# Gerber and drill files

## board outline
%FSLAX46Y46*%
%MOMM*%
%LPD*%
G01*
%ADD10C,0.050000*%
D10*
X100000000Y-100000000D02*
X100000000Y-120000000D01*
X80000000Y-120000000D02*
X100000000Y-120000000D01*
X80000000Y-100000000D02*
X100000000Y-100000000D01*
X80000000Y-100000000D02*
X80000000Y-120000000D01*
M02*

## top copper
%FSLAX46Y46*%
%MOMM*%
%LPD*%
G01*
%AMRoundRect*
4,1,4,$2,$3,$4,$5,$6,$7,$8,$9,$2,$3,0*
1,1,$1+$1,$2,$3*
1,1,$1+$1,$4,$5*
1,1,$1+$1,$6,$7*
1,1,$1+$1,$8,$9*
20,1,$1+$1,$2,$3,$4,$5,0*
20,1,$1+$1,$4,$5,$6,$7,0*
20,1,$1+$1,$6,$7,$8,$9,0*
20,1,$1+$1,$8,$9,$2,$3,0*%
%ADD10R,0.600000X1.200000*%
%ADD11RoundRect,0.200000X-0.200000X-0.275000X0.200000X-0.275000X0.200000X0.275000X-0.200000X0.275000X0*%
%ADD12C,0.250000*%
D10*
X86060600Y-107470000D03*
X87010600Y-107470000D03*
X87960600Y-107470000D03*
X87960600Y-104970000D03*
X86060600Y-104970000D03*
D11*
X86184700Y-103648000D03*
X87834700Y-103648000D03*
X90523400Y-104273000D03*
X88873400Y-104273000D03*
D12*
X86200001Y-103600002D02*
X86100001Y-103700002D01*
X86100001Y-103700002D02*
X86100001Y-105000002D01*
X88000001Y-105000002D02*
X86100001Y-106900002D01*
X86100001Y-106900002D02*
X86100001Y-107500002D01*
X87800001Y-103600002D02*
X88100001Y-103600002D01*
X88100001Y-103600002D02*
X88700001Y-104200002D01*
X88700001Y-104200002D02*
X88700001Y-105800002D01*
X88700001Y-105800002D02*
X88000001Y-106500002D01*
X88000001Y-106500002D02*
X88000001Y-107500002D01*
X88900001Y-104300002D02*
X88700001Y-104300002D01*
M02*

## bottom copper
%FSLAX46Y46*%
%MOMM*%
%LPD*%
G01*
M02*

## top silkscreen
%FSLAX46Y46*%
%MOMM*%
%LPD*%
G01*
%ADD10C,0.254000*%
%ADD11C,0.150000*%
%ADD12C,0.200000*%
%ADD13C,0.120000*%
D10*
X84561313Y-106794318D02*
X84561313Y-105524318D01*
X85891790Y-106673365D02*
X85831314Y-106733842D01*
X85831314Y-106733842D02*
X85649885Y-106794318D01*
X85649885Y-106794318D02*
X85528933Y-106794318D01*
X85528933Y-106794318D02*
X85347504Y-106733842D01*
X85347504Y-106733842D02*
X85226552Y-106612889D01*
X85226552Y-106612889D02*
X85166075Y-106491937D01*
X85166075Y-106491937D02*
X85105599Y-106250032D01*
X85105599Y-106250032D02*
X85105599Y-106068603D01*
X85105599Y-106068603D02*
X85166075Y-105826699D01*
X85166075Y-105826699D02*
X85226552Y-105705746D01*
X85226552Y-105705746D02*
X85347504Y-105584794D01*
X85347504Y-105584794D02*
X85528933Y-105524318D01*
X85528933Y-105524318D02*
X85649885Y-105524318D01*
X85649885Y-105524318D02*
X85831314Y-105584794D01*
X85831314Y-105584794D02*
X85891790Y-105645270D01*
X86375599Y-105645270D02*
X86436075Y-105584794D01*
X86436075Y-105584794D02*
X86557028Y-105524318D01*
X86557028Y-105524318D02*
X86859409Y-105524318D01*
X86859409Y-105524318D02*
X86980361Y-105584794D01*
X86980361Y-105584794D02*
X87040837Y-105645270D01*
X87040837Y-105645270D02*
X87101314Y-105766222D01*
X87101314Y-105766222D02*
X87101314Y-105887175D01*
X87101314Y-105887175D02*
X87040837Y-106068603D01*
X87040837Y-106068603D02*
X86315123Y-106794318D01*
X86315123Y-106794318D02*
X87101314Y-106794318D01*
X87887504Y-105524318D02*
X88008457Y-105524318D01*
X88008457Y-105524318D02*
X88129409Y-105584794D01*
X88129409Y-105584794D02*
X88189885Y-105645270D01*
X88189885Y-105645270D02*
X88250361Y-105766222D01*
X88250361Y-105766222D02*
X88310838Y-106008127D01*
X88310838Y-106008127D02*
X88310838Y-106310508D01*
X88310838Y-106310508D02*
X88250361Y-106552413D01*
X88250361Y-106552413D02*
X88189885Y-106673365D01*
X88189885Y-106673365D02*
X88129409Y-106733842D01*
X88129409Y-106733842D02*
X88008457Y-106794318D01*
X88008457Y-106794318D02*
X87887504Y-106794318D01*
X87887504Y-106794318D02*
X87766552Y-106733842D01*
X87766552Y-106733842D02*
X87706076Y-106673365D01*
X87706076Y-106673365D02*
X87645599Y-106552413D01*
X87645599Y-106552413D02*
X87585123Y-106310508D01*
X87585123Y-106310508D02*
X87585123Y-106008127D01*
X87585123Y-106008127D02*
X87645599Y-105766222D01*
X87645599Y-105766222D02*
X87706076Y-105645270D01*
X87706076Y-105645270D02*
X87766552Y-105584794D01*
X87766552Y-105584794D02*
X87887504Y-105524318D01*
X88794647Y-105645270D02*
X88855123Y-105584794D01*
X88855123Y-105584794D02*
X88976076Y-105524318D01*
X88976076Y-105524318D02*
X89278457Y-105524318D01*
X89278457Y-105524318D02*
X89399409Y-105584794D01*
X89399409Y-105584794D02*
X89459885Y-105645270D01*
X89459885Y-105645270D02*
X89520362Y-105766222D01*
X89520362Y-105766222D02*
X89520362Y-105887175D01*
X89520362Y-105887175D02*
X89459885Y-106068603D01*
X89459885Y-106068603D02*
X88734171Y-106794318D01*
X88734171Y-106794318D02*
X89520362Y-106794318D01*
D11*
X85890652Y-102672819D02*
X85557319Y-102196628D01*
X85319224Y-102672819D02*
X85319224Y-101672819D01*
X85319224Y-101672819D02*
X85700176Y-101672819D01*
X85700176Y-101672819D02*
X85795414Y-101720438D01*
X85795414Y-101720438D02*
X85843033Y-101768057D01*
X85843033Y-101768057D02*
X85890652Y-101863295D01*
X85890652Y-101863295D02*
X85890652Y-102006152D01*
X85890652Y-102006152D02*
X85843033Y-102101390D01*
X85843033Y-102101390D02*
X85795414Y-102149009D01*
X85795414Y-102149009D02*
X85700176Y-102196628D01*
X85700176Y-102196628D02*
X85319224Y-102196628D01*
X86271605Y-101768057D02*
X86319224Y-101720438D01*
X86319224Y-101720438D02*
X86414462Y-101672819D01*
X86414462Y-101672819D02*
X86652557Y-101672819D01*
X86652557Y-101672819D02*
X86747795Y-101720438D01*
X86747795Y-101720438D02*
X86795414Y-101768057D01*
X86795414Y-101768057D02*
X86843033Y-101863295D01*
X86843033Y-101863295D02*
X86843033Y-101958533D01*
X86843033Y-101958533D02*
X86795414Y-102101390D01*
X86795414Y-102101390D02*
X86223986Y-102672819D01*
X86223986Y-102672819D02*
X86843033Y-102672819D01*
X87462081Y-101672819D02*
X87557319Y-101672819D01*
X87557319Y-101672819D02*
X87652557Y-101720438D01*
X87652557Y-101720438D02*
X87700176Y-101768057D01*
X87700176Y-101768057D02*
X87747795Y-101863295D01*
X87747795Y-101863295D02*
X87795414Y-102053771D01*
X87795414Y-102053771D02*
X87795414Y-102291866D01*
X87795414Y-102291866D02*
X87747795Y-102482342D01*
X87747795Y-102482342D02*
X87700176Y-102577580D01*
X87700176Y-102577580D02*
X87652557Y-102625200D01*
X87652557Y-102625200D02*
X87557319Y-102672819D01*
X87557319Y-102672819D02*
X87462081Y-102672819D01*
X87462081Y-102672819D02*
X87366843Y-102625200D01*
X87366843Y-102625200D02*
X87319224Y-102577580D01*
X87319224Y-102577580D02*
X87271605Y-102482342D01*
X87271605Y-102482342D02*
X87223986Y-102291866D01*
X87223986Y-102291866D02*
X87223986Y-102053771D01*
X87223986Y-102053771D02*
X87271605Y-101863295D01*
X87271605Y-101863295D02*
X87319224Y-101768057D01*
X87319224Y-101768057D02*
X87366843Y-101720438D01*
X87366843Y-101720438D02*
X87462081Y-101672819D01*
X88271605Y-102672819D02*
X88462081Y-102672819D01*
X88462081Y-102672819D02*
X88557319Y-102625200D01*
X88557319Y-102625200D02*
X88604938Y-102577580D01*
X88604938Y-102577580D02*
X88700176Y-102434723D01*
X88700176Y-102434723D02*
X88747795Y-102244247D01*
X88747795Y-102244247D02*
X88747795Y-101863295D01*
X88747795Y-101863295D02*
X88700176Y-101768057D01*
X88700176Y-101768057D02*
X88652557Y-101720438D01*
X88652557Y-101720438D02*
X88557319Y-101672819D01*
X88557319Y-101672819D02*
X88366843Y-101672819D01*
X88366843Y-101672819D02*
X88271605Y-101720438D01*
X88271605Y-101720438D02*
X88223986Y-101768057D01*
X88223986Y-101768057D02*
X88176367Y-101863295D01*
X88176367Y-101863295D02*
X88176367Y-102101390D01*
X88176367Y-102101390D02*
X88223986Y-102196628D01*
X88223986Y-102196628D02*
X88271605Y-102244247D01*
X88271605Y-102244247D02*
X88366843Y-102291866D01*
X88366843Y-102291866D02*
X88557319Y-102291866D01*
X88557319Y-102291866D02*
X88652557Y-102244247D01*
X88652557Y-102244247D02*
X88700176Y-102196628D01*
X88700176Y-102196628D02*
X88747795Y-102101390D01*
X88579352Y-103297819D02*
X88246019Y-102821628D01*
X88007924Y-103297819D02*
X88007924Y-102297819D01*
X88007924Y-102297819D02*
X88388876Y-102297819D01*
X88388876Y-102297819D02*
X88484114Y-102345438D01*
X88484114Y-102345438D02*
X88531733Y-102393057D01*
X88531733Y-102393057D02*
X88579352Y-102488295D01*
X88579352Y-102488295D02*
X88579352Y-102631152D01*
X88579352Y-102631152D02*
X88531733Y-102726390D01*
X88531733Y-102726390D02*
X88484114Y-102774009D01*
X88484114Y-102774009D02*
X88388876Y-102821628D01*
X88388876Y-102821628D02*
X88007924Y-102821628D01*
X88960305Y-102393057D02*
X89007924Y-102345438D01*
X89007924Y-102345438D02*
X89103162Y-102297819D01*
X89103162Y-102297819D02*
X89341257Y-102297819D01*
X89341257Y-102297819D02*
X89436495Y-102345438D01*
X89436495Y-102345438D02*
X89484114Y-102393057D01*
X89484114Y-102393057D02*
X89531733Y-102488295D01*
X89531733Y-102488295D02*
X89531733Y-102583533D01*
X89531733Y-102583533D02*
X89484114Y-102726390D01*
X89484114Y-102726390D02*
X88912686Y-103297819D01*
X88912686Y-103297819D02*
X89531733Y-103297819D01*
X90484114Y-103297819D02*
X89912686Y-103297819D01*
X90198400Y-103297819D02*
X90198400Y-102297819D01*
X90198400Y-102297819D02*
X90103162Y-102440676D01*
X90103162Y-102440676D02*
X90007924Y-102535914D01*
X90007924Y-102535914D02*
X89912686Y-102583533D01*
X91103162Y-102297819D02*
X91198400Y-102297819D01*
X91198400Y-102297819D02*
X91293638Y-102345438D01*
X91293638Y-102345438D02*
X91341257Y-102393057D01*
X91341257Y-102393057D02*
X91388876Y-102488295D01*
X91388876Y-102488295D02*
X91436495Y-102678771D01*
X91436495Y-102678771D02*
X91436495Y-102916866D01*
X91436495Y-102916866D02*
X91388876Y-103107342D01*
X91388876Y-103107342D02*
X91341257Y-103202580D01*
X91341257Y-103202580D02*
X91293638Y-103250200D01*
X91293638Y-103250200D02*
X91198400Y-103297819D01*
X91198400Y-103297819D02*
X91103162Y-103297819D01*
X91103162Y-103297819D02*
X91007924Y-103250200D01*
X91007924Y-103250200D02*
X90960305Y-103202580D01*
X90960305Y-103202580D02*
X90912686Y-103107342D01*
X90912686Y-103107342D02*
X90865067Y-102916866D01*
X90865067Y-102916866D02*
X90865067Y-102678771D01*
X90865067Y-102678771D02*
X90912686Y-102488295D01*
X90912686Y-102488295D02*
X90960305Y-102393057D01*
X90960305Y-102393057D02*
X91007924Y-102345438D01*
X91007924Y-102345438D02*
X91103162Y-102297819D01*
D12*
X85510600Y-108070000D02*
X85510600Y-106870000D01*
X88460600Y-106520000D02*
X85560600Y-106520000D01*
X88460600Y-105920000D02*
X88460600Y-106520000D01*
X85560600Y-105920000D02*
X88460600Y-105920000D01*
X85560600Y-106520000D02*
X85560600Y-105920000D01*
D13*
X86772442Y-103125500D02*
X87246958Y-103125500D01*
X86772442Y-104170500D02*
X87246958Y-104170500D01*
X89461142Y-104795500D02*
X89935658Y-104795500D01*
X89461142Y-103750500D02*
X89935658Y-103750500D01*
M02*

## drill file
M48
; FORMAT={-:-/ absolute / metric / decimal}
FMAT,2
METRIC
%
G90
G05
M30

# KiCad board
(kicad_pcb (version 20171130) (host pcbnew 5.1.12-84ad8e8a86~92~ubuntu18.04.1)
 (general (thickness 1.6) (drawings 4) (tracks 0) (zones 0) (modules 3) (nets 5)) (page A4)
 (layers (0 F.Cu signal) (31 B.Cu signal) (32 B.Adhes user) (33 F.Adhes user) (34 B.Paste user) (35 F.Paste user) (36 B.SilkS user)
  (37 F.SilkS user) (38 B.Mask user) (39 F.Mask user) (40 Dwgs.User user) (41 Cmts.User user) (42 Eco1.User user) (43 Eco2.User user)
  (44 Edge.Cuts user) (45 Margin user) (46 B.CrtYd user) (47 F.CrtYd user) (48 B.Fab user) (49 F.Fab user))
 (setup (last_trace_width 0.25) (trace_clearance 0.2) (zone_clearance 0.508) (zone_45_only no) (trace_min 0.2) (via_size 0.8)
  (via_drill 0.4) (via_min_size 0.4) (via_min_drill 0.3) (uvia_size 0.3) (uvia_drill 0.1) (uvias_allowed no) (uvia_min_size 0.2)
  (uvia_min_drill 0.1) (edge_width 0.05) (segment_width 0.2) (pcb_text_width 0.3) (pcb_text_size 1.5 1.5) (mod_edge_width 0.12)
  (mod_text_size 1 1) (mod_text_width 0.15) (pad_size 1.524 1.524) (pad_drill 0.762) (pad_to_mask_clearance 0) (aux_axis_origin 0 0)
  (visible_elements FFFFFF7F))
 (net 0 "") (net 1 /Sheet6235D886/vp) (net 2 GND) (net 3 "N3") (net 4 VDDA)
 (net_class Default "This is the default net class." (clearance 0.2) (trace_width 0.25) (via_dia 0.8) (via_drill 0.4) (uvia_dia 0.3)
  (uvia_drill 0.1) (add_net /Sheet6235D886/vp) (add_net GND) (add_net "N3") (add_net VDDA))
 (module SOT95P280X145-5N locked (layer F.Cu) (at 87.010600 106.220000 90.000000)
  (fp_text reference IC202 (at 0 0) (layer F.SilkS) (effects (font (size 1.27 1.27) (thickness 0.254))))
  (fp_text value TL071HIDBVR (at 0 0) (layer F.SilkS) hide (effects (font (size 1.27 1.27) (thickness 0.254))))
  (fp_line (start -1.85 -1.5) (end -0.65 -1.5) (layer F.SilkS) (width 0.2))
  (fp_line (start -0.3 1.45) (end -0.3 -1.45) (layer F.SilkS) (width 0.2))
  (fp_line (start 0.3 1.45) (end -0.3 1.45) (layer F.SilkS) (width 0.2))
  (fp_line (start 0.3 -1.45) (end 0.3 1.45) (layer F.SilkS) (width 0.2))
  (fp_line (start -0.3 -1.45) (end 0.3 -1.45) (layer F.SilkS) (width 0.2))
  (pad 1 smd rect (at -1.25 -0.95 180.000000) (size 0.6 1.2) (layers F.Cu F.Mask F.Paste) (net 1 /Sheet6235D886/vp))
  (pad 2 smd rect (at -1.25 0 180.000000) (size 0.6 1.2) (layers F.Cu F.Mask F.Paste) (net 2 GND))
  (pad 3 smd rect (at -1.25 0.95 180.000000) (size 0.6 1.2) (layers F.Cu F.Mask F.Paste) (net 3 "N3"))
  (pad 4 smd rect (at 1.25 0.95 180.000000) (size 0.6 1.2) (layers F.Cu F.Mask F.Paste) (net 1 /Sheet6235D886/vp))
  (pad 5 smd rect (at 1.25 -0.95 180.000000) (size 0.6 1.2) (layers F.Cu F.Mask F.Paste) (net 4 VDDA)))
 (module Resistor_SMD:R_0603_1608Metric (layer F.Cu) (at 87.009700 103.648000)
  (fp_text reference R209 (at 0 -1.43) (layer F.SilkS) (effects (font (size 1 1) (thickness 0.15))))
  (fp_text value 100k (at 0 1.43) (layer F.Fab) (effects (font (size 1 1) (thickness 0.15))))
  (fp_line (start -0.237258 -0.5225) (end 0.237258 -0.5225) (layer F.SilkS) (width 0.12))
  (fp_line (start -0.237258 0.5225) (end 0.237258 0.5225) (layer F.SilkS) (width 0.12))
  (pad 1 smd roundrect (at -0.825 0) (size 0.8 0.95) (layers F.Cu F.Mask F.Paste) (roundrect_rratio 0.25) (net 4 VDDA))
  (pad 2 smd roundrect (at 0.825 0) (size 0.8 0.95) (layers F.Cu F.Mask F.Paste) (roundrect_rratio 0.25) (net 3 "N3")))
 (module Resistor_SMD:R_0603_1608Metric (layer F.Cu) (at 89.698400 104.273000)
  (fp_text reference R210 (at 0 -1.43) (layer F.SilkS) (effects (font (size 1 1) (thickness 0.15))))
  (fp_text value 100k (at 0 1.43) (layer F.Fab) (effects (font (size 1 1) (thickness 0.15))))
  (fp_line (start -0.237258 0.5225) (end 0.237258 0.5225) (layer F.SilkS) (width 0.12))
  (fp_line (start -0.237258 -0.5225) (end 0.237258 -0.5225) (layer F.SilkS) (width 0.12))
  (pad 2 smd roundrect (at 0.825 0) (size 0.8 0.95) (layers F.Cu F.Mask F.Paste) (roundrect_rratio 0.25) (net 2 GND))
  (pad 1 smd roundrect (at -0.825 0) (size 0.8 0.95) (layers F.Cu F.Mask F.Paste) (roundrect_rratio 0.25) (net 3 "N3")))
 (gr_line (start 100 100) (end 100 120) (layer Edge.Cuts) (width 0.05))
 (gr_line (start 80 120) (end 100 120) (layer Edge.Cuts) (width 0.05))
 (gr_line (start 80 100) (end 100 100) (layer Edge.Cuts) (width 0.05))
 (gr_line (start 80 100) (end 80 120) (layer Edge.Cuts) (width 0.05))
 (segment (start 86.200001 103.600002) (end 86.100001 103.700002) (width 0.250000) (layer F.Cu) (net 4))
 (segment (start 86.100001 103.700002) (end 86.100001 105.000002) (width 0.250000) (layer F.Cu) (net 4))
 (segment (start 88.000001 105.000002) (end 86.100001 106.900002) (width 0.250000) (layer F.Cu) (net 1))
 (segment (start 86.100001 106.900002) (end 86.100001 107.500002) (width 0.250000) (layer F.Cu) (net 1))
 (segment (start 87.800001 103.600002) (end 88.100001 103.600002) (width 0.250000) (layer F.Cu) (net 3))
 (segment (start 88.100001 103.600002) (end 88.700001 104.200002) (width 0.250000) (layer F.Cu) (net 3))
 (segment (start 88.700001 104.200002) (end 88.700001 105.800002) (width 0.250000) (layer F.Cu) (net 3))
 (segment (start 88.700001 105.800002) (end 88.000001 106.500002) (width 0.250000) (layer F.Cu) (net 3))
 (segment (start 88.000001 106.500002) (end 88.000001 107.500002) (width 0.250000) (layer F.Cu) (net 3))
 (segment (start 88.900001 104.300002) (end 88.700001 104.300002) (width 0.250000) (layer F.Cu) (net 3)))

